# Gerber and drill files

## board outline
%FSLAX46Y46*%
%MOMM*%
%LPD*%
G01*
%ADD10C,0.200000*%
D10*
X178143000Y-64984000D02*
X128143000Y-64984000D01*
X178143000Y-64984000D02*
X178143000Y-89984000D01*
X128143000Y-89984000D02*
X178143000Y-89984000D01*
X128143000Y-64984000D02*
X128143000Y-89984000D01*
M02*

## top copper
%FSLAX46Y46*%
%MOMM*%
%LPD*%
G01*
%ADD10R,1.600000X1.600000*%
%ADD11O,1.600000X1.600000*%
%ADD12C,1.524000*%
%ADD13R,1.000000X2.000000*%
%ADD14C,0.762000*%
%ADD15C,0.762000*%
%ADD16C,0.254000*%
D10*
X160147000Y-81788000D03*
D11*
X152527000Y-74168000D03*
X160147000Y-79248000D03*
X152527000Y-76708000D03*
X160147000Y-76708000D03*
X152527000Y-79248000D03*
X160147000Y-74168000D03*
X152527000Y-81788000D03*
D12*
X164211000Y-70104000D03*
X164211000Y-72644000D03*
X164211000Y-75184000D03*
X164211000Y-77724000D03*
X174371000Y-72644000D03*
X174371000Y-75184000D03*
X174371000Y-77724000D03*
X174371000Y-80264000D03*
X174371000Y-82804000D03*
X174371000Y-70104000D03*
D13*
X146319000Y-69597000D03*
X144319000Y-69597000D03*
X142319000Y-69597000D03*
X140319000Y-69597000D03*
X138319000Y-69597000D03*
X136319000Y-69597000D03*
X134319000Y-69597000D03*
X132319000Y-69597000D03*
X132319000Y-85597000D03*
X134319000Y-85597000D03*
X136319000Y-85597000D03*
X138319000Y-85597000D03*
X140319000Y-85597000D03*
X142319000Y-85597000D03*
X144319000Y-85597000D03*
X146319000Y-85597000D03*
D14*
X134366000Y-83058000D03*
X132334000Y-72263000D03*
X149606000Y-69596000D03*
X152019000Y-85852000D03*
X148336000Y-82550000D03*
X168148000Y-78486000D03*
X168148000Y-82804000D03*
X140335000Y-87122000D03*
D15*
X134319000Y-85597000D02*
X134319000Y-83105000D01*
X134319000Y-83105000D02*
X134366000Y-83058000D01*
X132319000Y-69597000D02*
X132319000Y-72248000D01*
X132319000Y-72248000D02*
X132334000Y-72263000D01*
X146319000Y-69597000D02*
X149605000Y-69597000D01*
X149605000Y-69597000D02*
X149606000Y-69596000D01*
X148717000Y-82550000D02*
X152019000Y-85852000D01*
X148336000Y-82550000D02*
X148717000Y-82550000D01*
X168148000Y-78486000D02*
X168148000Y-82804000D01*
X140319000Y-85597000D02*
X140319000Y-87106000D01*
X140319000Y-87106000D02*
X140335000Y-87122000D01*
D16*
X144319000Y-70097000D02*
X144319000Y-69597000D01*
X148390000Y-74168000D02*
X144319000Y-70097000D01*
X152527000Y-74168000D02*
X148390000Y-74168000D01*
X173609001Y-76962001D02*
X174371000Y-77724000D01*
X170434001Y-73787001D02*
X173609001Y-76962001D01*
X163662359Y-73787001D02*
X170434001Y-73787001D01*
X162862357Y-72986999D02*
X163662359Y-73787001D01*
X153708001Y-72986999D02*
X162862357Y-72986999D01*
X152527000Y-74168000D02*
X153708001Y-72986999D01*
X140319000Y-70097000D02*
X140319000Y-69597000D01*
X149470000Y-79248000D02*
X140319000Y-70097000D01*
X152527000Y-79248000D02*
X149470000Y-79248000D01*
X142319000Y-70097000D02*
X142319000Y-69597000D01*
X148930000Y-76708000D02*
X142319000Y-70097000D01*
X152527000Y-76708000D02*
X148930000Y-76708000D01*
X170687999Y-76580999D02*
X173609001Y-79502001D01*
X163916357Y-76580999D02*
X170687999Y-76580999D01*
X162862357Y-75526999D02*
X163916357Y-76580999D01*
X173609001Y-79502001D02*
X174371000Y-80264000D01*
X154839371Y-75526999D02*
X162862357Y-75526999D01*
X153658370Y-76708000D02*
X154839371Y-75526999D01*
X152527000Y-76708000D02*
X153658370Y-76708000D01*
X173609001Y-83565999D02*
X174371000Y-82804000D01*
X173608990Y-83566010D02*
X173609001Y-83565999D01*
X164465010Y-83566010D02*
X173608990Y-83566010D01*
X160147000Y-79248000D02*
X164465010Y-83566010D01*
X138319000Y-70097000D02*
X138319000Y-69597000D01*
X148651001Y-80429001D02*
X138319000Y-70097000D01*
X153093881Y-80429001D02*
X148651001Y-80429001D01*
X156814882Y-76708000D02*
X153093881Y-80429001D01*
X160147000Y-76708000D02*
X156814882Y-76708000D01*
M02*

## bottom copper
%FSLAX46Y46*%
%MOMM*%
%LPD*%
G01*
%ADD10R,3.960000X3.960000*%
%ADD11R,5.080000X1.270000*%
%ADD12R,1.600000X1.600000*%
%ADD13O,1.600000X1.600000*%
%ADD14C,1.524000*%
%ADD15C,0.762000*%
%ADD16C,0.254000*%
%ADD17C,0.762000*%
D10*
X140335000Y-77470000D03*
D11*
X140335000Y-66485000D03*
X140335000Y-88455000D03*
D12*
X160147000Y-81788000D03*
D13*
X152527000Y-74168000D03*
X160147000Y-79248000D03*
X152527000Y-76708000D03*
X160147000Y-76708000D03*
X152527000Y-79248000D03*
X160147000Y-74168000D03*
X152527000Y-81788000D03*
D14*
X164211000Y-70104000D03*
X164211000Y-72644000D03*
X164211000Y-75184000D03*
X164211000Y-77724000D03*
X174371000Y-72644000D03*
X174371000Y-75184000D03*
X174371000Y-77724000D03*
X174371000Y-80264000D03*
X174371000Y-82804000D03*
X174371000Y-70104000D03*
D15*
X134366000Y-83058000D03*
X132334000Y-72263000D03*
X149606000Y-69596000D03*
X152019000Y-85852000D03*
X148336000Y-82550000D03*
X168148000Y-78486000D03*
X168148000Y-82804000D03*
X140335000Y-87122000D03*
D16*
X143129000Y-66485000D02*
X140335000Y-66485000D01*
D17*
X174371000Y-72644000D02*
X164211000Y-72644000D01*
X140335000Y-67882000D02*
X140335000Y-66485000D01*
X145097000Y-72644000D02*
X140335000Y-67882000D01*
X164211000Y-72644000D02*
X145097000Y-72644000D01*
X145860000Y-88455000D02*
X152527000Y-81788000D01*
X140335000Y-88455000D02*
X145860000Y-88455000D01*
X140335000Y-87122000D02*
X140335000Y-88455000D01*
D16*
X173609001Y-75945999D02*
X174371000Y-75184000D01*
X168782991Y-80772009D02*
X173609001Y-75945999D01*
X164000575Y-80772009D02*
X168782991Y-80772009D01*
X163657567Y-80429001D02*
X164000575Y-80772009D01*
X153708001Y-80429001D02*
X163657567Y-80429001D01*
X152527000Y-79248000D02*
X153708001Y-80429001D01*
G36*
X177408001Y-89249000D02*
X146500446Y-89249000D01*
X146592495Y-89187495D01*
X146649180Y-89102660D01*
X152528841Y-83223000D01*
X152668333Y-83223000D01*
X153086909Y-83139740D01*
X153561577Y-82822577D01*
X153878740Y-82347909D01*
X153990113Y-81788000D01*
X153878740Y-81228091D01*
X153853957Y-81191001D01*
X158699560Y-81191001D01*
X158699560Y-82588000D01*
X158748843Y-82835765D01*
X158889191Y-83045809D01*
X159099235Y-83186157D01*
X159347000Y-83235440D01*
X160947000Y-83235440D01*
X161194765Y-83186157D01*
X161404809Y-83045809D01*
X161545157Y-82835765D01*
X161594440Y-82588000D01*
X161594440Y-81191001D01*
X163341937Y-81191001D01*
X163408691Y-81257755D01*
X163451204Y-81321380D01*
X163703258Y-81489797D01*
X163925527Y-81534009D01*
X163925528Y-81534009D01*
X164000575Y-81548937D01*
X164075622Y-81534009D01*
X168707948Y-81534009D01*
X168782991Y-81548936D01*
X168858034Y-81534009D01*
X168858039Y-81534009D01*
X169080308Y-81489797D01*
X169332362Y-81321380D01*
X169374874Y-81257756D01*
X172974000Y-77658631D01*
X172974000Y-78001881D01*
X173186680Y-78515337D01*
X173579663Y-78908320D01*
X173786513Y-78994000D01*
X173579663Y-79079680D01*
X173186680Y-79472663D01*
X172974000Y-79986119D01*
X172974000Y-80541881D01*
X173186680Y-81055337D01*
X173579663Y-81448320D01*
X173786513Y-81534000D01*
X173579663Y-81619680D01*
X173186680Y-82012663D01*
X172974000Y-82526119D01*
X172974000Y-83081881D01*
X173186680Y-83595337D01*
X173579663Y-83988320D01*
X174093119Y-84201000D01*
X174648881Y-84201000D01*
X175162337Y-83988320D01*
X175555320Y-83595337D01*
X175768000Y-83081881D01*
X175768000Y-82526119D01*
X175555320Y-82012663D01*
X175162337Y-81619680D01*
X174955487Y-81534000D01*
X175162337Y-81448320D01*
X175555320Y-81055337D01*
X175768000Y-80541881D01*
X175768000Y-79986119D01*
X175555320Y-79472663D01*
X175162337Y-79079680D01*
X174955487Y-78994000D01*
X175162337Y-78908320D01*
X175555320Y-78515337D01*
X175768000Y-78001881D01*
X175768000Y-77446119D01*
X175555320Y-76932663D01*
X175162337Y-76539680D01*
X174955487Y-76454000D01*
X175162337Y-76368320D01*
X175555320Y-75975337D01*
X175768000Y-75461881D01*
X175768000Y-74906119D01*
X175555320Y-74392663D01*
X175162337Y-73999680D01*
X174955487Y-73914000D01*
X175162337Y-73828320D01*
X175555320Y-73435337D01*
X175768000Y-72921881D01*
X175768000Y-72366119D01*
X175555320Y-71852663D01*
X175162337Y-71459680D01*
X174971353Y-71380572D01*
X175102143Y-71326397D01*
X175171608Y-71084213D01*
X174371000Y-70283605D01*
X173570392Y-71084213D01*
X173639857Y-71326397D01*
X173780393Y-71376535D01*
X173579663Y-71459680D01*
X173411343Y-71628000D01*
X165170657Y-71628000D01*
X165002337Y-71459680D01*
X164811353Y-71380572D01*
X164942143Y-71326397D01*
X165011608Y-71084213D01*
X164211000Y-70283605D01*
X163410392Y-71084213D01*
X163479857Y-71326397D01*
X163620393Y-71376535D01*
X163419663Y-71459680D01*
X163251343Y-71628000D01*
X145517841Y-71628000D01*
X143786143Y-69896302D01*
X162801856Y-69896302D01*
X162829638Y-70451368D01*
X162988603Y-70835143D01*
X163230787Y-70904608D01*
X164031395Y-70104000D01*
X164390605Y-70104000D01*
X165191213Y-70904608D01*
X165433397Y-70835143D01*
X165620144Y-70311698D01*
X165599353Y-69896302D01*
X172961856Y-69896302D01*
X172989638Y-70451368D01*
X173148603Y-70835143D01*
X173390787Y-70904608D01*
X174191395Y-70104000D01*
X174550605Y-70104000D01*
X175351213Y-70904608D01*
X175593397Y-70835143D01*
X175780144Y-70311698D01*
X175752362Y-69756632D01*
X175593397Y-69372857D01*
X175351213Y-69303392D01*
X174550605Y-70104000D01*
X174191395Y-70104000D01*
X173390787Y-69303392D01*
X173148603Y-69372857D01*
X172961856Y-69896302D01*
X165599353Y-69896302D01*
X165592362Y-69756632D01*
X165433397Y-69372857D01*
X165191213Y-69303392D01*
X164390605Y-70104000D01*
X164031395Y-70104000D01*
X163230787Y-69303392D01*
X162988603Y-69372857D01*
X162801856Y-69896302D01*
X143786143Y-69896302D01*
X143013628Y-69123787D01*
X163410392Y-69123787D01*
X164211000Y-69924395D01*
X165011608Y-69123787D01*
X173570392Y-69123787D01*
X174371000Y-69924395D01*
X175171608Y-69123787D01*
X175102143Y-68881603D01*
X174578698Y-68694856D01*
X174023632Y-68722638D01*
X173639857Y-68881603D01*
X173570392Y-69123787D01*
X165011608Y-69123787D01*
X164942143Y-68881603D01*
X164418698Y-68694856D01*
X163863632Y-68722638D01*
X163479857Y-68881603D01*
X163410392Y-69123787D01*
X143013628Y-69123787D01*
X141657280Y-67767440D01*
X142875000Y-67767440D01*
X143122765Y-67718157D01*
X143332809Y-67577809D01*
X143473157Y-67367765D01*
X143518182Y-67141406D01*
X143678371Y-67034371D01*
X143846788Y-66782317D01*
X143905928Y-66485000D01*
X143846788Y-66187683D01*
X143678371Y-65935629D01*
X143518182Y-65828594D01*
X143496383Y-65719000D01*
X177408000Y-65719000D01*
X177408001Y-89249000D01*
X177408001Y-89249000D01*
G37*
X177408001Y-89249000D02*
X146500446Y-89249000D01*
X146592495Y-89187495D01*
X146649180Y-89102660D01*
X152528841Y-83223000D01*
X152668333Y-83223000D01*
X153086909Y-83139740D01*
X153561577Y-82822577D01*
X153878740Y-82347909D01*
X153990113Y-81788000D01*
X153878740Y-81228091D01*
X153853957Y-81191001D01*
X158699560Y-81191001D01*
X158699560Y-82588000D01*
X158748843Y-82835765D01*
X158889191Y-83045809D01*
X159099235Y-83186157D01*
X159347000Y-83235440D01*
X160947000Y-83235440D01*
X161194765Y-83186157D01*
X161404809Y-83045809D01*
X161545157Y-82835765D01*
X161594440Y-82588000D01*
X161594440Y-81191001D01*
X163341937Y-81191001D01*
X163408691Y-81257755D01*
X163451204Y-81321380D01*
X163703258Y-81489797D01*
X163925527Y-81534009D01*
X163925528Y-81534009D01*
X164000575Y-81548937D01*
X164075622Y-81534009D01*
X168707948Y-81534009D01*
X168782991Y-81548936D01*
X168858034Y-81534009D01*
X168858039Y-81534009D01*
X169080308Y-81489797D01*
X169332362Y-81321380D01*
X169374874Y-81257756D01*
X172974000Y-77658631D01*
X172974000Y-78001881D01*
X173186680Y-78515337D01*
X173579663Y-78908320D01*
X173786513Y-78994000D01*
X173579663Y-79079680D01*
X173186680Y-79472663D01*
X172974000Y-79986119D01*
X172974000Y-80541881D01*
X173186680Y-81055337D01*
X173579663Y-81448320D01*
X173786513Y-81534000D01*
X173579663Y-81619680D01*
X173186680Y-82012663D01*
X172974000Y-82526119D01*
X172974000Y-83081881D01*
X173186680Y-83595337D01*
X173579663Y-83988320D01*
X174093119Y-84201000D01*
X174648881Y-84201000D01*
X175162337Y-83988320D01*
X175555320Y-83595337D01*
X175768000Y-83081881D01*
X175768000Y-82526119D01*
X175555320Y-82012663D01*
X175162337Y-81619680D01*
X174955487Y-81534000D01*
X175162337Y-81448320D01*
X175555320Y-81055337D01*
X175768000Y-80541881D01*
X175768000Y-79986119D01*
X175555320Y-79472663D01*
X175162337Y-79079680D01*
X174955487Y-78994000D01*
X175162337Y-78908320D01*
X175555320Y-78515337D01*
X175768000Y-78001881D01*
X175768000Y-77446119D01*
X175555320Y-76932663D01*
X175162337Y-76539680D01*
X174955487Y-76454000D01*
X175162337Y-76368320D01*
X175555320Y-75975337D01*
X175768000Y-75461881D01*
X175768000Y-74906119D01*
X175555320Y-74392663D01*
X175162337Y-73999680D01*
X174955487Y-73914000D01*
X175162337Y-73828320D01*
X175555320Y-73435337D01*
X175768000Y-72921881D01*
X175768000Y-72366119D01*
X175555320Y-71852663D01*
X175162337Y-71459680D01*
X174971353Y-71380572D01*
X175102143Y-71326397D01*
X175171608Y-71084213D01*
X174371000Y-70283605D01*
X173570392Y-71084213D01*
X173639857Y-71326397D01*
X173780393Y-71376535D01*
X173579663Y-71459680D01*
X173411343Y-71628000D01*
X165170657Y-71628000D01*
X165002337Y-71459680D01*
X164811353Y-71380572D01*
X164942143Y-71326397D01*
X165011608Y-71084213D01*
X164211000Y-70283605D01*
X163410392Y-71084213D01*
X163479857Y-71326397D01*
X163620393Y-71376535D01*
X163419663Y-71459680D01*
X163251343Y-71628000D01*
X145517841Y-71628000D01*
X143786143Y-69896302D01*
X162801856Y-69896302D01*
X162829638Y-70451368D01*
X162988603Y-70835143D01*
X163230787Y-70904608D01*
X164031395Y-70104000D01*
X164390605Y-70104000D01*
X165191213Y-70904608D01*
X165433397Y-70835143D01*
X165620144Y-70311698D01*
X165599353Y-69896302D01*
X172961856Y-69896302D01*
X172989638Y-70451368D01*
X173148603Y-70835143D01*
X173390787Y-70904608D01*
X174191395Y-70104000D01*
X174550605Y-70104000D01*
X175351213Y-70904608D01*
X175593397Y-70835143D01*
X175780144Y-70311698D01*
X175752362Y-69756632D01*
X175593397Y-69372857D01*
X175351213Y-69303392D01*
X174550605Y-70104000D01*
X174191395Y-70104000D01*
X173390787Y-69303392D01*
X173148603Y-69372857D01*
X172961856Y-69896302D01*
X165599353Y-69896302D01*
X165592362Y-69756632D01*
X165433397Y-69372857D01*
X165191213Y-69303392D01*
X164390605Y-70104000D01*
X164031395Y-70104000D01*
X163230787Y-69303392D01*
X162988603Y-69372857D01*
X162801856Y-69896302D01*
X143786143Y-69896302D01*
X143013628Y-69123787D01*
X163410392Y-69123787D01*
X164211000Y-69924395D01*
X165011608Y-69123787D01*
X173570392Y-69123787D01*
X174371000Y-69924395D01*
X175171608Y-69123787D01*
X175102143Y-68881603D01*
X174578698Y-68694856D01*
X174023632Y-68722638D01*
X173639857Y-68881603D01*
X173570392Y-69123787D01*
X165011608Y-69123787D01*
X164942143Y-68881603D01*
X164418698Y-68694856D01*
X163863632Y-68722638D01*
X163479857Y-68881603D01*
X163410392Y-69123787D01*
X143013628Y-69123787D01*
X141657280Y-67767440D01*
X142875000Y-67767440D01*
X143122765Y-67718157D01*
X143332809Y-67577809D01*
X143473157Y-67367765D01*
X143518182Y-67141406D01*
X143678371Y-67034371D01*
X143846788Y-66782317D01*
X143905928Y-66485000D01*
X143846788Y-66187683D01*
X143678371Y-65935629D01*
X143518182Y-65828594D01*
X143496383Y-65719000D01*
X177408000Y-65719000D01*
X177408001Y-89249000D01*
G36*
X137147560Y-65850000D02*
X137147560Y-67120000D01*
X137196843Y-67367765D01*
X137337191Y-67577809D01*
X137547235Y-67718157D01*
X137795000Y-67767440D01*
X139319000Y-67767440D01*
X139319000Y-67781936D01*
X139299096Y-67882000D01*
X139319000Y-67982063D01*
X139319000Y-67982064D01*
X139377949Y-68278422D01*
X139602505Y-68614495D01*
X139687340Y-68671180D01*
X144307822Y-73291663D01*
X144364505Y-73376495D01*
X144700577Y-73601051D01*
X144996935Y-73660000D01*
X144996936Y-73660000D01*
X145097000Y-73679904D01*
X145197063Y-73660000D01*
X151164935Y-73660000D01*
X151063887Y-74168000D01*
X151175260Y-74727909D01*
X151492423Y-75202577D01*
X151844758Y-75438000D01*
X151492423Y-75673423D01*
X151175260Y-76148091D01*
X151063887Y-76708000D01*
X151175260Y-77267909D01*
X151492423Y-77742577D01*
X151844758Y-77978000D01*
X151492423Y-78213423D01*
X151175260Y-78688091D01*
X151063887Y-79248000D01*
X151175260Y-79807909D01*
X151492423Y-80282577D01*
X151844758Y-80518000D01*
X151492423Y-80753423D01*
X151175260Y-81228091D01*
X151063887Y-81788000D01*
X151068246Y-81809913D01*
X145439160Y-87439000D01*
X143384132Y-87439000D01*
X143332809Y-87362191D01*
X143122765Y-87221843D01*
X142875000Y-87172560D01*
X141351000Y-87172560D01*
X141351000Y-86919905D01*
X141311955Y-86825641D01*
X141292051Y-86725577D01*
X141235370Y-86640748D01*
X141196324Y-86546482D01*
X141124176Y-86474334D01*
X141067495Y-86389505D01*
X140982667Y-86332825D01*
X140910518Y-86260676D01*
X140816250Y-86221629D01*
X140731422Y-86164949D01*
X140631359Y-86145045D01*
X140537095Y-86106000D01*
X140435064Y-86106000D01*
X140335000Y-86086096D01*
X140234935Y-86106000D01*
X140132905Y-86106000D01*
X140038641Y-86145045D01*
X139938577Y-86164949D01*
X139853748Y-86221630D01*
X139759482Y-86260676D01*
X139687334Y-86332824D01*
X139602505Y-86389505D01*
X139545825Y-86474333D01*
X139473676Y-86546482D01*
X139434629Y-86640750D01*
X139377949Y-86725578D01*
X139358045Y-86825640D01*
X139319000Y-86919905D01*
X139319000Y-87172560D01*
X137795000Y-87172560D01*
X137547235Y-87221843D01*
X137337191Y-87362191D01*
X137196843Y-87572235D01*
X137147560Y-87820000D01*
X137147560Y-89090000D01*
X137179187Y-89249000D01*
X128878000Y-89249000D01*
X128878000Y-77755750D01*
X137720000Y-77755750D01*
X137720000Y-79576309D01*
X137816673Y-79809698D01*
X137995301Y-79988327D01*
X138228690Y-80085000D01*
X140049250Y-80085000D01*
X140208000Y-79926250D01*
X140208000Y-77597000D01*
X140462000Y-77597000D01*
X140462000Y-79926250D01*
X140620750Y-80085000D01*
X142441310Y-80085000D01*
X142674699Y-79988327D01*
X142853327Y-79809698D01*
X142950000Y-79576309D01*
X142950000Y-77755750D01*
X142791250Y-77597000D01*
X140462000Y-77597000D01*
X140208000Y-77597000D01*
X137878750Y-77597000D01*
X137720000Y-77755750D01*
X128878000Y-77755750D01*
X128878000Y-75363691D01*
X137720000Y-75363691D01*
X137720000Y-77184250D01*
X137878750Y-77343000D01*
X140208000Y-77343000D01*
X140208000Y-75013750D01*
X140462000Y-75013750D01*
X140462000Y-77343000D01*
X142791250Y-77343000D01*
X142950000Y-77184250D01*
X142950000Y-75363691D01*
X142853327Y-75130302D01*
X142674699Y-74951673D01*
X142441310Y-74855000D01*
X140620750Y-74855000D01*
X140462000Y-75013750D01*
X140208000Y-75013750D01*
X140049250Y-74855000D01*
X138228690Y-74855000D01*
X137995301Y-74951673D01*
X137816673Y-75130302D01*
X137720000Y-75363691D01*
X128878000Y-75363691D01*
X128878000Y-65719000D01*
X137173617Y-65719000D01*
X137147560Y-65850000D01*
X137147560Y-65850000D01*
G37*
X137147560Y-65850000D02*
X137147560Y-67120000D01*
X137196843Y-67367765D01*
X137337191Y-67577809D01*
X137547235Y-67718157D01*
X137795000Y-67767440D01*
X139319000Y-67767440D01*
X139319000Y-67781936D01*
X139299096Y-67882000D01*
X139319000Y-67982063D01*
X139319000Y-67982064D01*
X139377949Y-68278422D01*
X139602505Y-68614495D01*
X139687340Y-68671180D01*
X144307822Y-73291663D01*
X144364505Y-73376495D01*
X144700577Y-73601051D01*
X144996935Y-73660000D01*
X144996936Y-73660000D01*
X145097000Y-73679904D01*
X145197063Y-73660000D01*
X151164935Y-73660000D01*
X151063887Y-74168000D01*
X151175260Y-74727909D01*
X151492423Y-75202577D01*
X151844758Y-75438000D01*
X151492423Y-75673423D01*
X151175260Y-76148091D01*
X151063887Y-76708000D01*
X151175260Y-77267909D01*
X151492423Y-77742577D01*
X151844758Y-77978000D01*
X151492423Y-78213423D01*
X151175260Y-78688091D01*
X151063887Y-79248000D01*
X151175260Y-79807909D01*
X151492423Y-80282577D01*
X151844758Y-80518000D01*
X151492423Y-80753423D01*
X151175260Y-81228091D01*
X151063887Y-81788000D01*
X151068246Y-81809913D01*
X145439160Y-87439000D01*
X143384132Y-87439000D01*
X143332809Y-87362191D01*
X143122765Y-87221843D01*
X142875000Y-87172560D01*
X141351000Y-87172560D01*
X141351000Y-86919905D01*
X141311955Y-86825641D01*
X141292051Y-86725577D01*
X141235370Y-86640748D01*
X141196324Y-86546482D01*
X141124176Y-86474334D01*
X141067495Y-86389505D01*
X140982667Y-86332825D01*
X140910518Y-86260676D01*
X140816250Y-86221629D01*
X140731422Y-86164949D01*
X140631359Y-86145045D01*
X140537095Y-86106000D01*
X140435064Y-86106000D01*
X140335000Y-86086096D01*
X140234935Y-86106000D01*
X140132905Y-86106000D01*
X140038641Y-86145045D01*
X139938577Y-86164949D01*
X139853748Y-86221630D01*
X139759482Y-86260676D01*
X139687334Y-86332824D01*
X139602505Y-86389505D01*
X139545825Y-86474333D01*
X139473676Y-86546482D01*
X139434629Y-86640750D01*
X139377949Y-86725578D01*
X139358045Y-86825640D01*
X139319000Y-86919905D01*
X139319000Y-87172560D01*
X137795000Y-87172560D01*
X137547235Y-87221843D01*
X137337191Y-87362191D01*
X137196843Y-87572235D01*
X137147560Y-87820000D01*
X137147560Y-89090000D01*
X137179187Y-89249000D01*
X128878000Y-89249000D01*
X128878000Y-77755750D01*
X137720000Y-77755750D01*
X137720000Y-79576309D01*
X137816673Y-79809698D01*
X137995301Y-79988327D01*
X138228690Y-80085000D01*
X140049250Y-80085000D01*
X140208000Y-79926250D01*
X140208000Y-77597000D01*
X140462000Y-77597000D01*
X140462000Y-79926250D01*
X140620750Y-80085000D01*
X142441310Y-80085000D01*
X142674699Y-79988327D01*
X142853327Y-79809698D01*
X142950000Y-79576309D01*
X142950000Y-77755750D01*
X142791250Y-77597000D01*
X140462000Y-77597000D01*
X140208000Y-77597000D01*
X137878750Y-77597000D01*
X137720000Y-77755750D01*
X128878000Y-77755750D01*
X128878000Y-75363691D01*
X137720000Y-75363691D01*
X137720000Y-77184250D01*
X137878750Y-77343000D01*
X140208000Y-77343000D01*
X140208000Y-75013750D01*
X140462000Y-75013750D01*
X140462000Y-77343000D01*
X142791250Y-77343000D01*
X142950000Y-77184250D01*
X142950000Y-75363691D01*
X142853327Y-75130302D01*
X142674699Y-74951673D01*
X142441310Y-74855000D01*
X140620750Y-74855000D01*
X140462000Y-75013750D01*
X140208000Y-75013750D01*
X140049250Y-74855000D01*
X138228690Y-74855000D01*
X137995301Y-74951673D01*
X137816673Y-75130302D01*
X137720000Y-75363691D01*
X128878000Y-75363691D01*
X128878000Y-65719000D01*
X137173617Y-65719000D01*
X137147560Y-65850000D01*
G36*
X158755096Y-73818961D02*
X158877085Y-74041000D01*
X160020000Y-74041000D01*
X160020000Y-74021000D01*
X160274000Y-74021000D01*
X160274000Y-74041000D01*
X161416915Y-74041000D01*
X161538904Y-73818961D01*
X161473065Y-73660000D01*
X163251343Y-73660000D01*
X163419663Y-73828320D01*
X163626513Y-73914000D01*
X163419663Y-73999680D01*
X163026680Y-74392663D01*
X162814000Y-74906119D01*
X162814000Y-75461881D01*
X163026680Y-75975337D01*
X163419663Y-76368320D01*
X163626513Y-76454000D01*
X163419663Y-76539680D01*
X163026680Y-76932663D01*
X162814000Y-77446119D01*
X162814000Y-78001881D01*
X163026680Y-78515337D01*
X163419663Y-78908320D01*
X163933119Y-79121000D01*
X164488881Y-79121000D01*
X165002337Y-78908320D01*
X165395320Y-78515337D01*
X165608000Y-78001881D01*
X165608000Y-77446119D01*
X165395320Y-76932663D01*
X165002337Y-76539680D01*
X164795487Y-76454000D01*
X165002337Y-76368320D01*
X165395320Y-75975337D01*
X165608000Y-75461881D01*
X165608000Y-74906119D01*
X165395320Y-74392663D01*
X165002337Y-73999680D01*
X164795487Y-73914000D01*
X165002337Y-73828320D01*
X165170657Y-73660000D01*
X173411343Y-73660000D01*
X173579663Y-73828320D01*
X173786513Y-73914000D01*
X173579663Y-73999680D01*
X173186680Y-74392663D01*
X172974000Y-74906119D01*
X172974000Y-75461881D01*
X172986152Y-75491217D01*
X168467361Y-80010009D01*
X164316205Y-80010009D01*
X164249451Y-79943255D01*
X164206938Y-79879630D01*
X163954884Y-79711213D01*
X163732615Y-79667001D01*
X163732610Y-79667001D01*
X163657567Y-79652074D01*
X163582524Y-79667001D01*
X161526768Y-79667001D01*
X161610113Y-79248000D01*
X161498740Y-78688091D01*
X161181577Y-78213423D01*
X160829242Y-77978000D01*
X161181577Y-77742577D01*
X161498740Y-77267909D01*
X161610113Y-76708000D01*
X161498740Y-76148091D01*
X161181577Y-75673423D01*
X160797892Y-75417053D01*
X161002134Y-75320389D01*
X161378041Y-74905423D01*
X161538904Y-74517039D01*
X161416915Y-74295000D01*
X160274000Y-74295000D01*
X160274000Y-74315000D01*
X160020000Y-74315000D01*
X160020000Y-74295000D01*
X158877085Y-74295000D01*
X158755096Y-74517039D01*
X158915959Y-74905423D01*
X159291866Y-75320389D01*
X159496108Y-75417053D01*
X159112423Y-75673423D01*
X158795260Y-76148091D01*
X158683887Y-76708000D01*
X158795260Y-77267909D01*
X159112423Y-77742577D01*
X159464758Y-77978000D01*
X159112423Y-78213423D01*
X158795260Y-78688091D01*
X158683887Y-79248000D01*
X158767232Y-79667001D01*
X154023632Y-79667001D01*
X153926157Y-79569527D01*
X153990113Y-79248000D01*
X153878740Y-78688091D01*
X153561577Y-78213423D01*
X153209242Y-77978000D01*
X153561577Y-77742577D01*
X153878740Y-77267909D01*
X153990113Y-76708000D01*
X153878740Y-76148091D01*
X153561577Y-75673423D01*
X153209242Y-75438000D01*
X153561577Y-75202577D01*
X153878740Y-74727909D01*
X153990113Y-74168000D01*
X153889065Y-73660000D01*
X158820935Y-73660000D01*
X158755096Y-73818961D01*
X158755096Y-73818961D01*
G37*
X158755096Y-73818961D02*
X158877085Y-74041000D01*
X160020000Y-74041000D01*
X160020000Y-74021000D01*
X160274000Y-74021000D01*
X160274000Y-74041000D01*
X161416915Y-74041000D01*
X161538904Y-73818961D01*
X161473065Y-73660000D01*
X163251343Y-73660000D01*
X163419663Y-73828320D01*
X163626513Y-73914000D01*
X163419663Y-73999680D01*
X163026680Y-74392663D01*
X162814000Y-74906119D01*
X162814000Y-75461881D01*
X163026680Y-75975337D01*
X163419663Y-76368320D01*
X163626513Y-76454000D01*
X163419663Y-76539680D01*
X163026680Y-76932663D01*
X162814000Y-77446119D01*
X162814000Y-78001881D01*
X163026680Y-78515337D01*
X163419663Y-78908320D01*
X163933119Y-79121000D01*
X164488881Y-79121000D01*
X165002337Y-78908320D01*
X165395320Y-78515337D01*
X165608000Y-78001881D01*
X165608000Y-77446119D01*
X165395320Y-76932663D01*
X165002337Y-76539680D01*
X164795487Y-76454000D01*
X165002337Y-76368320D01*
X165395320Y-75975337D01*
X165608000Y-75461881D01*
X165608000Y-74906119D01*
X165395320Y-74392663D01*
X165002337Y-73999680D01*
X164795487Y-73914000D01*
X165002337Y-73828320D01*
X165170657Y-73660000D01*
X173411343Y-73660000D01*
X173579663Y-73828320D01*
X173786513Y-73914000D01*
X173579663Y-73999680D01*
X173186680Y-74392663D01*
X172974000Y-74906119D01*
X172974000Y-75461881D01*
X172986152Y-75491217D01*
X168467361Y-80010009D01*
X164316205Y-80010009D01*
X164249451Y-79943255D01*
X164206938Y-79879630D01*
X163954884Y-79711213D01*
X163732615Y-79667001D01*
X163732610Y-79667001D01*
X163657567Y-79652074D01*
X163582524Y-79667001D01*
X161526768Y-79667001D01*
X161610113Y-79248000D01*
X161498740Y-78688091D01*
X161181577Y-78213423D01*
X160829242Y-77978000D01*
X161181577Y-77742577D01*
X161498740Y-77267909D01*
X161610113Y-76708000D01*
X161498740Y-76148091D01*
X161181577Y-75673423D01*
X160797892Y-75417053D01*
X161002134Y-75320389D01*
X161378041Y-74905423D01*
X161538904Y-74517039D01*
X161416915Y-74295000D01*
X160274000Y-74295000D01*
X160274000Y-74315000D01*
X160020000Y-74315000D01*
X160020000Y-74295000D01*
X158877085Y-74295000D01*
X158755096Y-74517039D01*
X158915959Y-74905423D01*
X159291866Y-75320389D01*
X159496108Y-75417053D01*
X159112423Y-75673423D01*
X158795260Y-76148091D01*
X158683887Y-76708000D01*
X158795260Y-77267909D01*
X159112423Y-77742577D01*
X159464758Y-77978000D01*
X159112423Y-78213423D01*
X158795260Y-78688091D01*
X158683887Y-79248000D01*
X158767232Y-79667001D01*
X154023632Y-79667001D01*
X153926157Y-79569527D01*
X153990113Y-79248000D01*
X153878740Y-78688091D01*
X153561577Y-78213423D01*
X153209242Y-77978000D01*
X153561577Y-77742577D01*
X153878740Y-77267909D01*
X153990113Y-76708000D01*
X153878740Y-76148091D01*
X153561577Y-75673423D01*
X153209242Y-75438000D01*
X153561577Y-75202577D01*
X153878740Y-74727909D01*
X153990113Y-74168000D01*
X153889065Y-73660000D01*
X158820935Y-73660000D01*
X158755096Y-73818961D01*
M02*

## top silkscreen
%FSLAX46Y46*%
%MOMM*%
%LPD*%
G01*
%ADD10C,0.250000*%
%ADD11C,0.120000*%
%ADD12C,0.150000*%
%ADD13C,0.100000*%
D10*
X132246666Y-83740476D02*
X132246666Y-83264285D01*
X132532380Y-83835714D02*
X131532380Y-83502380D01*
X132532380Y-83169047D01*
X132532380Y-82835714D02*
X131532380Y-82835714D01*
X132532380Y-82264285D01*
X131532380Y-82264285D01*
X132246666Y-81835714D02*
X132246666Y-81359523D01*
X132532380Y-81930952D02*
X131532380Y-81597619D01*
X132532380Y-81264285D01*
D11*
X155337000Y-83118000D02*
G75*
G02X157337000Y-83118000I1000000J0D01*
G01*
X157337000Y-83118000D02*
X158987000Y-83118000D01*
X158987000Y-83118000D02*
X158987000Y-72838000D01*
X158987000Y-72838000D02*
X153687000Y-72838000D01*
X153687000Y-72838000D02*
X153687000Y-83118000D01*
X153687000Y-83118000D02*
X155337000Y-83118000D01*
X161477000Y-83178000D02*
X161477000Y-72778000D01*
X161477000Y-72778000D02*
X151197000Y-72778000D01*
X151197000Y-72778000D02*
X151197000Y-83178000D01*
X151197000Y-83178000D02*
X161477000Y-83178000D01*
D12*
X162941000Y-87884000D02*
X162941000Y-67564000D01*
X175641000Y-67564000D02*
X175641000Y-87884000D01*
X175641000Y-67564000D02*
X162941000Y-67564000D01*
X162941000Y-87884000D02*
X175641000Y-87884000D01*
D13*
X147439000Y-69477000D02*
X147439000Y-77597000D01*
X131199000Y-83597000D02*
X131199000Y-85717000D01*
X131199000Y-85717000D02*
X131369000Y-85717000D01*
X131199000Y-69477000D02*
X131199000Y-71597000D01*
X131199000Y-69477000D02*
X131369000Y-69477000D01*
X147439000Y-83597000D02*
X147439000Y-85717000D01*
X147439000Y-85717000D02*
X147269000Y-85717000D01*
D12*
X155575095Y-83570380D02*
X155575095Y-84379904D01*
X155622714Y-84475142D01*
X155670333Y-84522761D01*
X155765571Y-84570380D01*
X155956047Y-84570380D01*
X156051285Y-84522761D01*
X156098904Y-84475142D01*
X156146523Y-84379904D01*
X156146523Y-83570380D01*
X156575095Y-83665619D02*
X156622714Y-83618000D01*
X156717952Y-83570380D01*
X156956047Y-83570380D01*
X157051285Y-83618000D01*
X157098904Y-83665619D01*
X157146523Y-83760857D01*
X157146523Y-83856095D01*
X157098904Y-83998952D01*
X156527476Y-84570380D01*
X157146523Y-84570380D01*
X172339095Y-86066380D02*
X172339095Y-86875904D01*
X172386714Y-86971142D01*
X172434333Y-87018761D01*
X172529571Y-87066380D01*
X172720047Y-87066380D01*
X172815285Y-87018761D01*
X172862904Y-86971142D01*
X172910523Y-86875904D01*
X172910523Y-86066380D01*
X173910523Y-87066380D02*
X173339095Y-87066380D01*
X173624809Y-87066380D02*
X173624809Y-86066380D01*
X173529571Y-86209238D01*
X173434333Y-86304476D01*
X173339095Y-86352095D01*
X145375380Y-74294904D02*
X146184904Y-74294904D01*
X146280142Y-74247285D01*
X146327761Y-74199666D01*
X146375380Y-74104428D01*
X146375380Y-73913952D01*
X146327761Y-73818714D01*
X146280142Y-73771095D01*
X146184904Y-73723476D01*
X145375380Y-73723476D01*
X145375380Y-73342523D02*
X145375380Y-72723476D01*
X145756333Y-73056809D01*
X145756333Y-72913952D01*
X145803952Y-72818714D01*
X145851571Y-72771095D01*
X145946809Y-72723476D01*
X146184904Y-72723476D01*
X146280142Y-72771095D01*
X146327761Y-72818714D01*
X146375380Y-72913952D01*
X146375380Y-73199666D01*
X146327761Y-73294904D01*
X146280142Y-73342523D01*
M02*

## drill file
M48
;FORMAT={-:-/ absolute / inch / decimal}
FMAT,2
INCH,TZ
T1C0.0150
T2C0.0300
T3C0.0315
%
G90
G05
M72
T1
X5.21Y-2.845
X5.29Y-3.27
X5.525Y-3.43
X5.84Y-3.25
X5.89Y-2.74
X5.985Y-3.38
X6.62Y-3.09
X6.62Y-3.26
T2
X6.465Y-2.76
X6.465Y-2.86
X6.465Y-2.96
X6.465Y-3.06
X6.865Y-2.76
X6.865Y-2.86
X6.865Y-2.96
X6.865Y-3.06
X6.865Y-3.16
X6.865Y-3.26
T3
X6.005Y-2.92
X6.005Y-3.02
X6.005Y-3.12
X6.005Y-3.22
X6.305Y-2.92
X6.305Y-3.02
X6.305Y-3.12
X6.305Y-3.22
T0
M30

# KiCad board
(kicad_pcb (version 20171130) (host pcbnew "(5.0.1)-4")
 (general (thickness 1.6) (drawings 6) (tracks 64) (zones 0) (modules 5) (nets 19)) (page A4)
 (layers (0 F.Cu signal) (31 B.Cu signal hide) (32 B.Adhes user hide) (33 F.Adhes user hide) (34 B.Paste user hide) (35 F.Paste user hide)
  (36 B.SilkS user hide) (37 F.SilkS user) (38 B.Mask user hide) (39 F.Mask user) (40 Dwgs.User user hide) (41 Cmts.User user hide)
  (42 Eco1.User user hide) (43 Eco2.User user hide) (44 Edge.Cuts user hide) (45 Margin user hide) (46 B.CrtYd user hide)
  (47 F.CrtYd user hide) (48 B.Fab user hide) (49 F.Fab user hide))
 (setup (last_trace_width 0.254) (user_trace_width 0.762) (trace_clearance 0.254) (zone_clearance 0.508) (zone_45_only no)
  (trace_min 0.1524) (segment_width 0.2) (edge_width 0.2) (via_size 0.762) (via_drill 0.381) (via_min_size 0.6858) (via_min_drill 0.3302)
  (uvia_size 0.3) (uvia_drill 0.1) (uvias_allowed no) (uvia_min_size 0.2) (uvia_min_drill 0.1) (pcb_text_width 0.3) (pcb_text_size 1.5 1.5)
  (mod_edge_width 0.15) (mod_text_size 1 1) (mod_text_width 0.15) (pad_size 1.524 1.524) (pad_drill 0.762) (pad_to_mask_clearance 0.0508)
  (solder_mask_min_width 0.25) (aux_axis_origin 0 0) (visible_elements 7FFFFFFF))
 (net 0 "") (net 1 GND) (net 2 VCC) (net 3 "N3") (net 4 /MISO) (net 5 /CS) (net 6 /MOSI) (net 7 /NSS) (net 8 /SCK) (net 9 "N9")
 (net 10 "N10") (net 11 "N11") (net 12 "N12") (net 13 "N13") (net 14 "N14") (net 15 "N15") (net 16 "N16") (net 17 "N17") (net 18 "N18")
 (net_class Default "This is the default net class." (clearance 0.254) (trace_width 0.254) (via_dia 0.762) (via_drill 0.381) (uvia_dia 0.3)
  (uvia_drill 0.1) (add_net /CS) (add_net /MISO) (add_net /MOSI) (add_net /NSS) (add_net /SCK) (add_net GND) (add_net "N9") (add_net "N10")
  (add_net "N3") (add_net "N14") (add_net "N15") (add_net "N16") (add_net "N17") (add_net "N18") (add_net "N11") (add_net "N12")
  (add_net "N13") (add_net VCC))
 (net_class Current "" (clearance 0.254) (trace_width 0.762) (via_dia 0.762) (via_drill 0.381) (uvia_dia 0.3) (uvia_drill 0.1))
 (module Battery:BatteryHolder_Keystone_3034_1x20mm (layer B.Cu) (at 140.335 77.47 90)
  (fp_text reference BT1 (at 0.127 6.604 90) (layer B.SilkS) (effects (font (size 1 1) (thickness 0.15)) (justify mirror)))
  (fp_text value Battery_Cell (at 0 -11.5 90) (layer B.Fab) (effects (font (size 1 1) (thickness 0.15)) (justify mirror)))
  (pad 2 smd rect (at 0 0 90) (size 3.96 3.96) (layers B.Cu B.Paste B.Mask) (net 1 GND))
  (pad 1 smd rect (at 10.985 0 90) (size 1.27 5.08) (layers B.Cu B.Paste B.Mask) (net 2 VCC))
  (pad 1 smd rect (at -10.985 0 90) (size 1.27 5.08) (layers B.Cu B.Paste B.Mask) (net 2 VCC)))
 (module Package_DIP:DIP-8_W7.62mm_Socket (layer F.Cu) (at 160.147 81.788 180)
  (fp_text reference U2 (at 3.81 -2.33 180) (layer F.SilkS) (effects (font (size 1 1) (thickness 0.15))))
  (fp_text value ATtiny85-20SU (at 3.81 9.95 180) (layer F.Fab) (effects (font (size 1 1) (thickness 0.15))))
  (fp_arc (start 3.81 -1.33) (end 2.81 -1.33) (angle -180) (layer F.SilkS) (width 0.12))
  (fp_line (start 2.81 -1.33) (end 1.16 -1.33) (layer F.SilkS) (width 0.12))
  (fp_line (start 1.16 -1.33) (end 1.16 8.95) (layer F.SilkS) (width 0.12))
  (fp_line (start 1.16 8.95) (end 6.46 8.95) (layer F.SilkS) (width 0.12))
  (fp_line (start 6.46 8.95) (end 6.46 -1.33) (layer F.SilkS) (width 0.12))
  (fp_line (start 6.46 -1.33) (end 4.81 -1.33) (layer F.SilkS) (width 0.12))
  (fp_line (start -1.33 -1.39) (end -1.33 9.01) (layer F.SilkS) (width 0.12))
  (fp_line (start -1.33 9.01) (end 8.95 9.01) (layer F.SilkS) (width 0.12))
  (fp_line (start 8.95 9.01) (end 8.95 -1.39) (layer F.SilkS) (width 0.12))
  (fp_line (start 8.95 -1.39) (end -1.33 -1.39) (layer F.SilkS) (width 0.12))
  (pad 1 thru_hole rect (at 0 0 180) (size 1.6 1.6) (drill 0.8) (layers *.Cu *.Mask) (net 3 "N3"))
  (pad 5 thru_hole oval (at 7.62 7.62 180) (size 1.6 1.6) (drill 0.8) (layers *.Cu *.Mask) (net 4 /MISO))
  (pad 2 thru_hole oval (at 0 2.54 180) (size 1.6 1.6) (drill 0.8) (layers *.Cu *.Mask) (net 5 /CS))
  (pad 6 thru_hole oval (at 7.62 5.08 180) (size 1.6 1.6) (drill 0.8) (layers *.Cu *.Mask) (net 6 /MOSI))
  (pad 3 thru_hole oval (at 0 5.08 180) (size 1.6 1.6) (drill 0.8) (layers *.Cu *.Mask) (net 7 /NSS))
  (pad 7 thru_hole oval (at 7.62 2.54 180) (size 1.6 1.6) (drill 0.8) (layers *.Cu *.Mask) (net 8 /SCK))
  (pad 4 thru_hole oval (at 0 7.62 180) (size 1.6 1.6) (drill 0.8) (layers *.Cu *.Mask) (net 1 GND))
  (pad 8 thru_hole oval (at 7.62 0 180) (size 1.6 1.6) (drill 0.8) (layers *.Cu *.Mask) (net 2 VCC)))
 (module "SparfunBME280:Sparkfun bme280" (layer F.Cu) (at 169.291 77.724)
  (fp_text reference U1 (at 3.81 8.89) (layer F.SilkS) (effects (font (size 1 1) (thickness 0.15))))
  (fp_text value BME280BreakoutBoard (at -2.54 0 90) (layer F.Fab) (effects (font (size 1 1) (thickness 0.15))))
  (fp_line (start -6.35 10.16) (end -6.35 -10.16) (layer F.SilkS) (width 0.15))
  (fp_line (start 6.35 -10.16) (end 6.35 10.16) (layer F.SilkS) (width 0.15))
  (fp_line (start 6.35 -10.16) (end -6.35 -10.16) (layer F.SilkS) (width 0.15))
  (fp_line (start -6.35 10.16) (end 6.35 10.16) (layer F.SilkS) (width 0.15))
  (pad 1 thru_hole circle (at -5.08 -7.62) (size 1.524 1.524) (drill 0.762) (layers *.Cu *.Mask) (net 1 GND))
  (pad 2 thru_hole circle (at -5.08 -5.08) (size 1.524 1.524) (drill 0.762) (layers *.Cu *.Mask) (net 2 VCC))
  (pad 3 thru_hole circle (at -5.08 -2.54) (size 1.524 1.524) (drill 0.762) (layers *.Cu *.Mask) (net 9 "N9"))
  (pad 4 thru_hole circle (at -5.08 0) (size 1.524 1.524) (drill 0.762) (layers *.Cu *.Mask) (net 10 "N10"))
  (pad 6 thru_hole circle (at 5.08 -5.08) (size 1.524 1.524) (drill 0.762) (layers *.Cu *.Mask) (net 2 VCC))
  (pad 7 thru_hole circle (at 5.08 -2.54) (size 1.524 1.524) (drill 0.762) (layers *.Cu *.Mask) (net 8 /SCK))
  (pad 8 thru_hole circle (at 5.08 0) (size 1.524 1.524) (drill 0.762) (layers *.Cu *.Mask) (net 4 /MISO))
  (pad 9 thru_hole circle (at 5.08 2.54) (size 1.524 1.524) (drill 0.762) (layers *.Cu *.Mask) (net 6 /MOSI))
  (pad 10 thru_hole circle (at 5.08 5.08) (size 1.524 1.524) (drill 0.762) (layers *.Cu *.Mask) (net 5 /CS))
  (pad 5 thru_hole circle (at 5.08 -7.62) (size 1.524 1.524) (drill 0.762) (layers *.Cu *.Mask) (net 1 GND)))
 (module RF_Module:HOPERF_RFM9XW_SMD (layer F.Cu) (at 139.319 77.597 270)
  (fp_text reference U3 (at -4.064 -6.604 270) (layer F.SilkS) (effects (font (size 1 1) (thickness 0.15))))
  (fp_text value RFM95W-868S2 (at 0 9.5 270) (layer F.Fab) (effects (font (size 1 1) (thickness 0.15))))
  (fp_line (start -8.12 -8.12) (end 0 -8.12) (layer F.SilkS) (width 0.1))
  (fp_line (start 6 8.12) (end 8.12 8.12) (layer F.SilkS) (width 0.1))
  (fp_line (start 8.12 8.12) (end 8.12 7.95) (layer F.SilkS) (width 0.1))
  (fp_line (start -8.12 8.12) (end -6 8.12) (layer F.SilkS) (width 0.1))
  (fp_line (start -8.12 8.12) (end -8.12 7.95) (layer F.SilkS) (width 0.1))
  (fp_line (start 6 -8.12) (end 8.12 -8.12) (layer F.SilkS) (width 0.1))
  (fp_line (start 8.12 -8.12) (end 8.12 -7.95) (layer F.SilkS) (width 0.1))
  (pad 1 smd rect (at -8 -7 270) (size 2 1) (layers F.Cu F.Paste F.Mask) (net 1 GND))
  (pad 2 smd rect (at -8 -5 270) (size 2 1) (layers F.Cu F.Paste F.Mask) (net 4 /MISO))
  (pad 3 smd rect (at -8 -3 270) (size 2 1) (layers F.Cu F.Paste F.Mask) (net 6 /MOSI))
  (pad 4 smd rect (at -8 -1 270) (size 2 1) (layers F.Cu F.Paste F.Mask) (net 8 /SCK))
  (pad 5 smd rect (at -8 1 270) (size 2 1) (layers F.Cu F.Paste F.Mask) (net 7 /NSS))
  (pad 6 smd rect (at -8 3 270) (size 2 1) (layers F.Cu F.Paste F.Mask) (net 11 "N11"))
  (pad 7 smd rect (at -8 5 270) (size 2 1) (layers F.Cu F.Paste F.Mask) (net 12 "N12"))
  (pad 8 smd rect (at -8 7 270) (size 2 1) (layers F.Cu F.Paste F.Mask) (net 1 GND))
  (pad 9 smd rect (at 8 7 270) (size 2 1) (layers F.Cu F.Paste F.Mask) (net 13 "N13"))
  (pad 10 smd rect (at 8 5 270) (size 2 1) (layers F.Cu F.Paste F.Mask) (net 1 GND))
  (pad 11 smd rect (at 8 3 270) (size 2 1) (layers F.Cu F.Paste F.Mask) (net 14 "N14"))
  (pad 12 smd rect (at 8 1 270) (size 2 1) (layers F.Cu F.Paste F.Mask) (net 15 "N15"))
  (pad 13 smd rect (at 8 -1 270) (size 2 1) (layers F.Cu F.Paste F.Mask) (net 2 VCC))
  (pad 14 smd rect (at 8 -3 270) (size 2 1) (layers F.Cu F.Paste F.Mask) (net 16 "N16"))
  (pad 15 smd rect (at 8 -5 270) (size 2 1) (layers F.Cu F.Paste F.Mask) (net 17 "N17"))
  (pad 16 smd rect (at 8 -7 270) (size 2 1) (layers F.Cu F.Paste F.Mask) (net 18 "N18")))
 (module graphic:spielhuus (layer B.Cu) (at 171.069 68.072 270)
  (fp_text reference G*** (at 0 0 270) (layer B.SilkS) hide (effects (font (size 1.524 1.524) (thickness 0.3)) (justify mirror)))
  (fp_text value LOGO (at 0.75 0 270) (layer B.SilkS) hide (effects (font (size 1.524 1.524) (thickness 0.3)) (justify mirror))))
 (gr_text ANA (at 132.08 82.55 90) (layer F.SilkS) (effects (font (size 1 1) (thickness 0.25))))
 (gr_line (start 178.143 64.984) (end 128.143 64.984) (layer Edge.Cuts) (width 0.2))
 (gr_line (start 178.143 64.984) (end 178.143 89.984) (layer Edge.Cuts) (width 0.2))
 (gr_line (start 128.143 89.984) (end 178.143 89.984) (layer Edge.Cuts) (width 0.2))
 (gr_line (start 128.143 64.984) (end 128.143 89.984) (layer Edge.Cuts) (width 0.2))
 (via (at 134.366 83.058) (size 0.762) (drill 0.381) (layers F.Cu B.Cu) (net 1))
 (segment (start 134.319 85.597) (end 134.319 83.105) (width 0.762) (layer F.Cu) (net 1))
 (segment (start 134.319 83.105) (end 134.366 83.058) (width 0.762) (layer F.Cu) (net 1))
 (via (at 132.334 72.263) (size 0.762) (drill 0.381) (layers F.Cu B.Cu) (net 1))
 (segment (start 132.319 69.597) (end 132.319 72.248) (width 0.762) (layer F.Cu) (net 1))
 (segment (start 132.319 72.248) (end 132.334 72.263) (width 0.762) (layer F.Cu) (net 1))
 (via (at 149.606 69.596) (size 0.762) (drill 0.381) (layers F.Cu B.Cu) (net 1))
 (segment (start 146.319 69.597) (end 149.605 69.597) (width 0.762) (layer F.Cu) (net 1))
 (segment (start 149.605 69.597) (end 149.606 69.596) (width 0.762) (layer F.Cu) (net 1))
 (via (at 152.019 85.852) (size 0.762) (drill 0.381) (layers F.Cu B.Cu) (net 1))
 (via (at 148.336 82.55) (size 0.762) (drill 0.381) (layers F.Cu B.Cu) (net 1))
 (segment (start 148.717 82.55) (end 152.019 85.852) (width 0.762) (layer F.Cu) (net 1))
 (segment (start 148.336 82.55) (end 148.717 82.55) (width 0.762) (layer F.Cu) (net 1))
 (via (at 168.148 78.486) (size 0.762) (drill 0.381) (layers F.Cu B.Cu) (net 1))
 (via (at 168.148 82.804) (size 0.762) (drill 0.381) (layers F.Cu B.Cu) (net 1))
 (segment (start 168.148 78.486) (end 168.148 82.804) (width 0.762) (layer F.Cu) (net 1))
 (segment (start 143.129 66.485) (end 140.335 66.485) (width 0.254) (layer B.Cu) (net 2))
 (segment (start 174.371 72.644) (end 164.211 72.644) (width 0.762) (layer B.Cu) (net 2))
 (segment (start 140.335 67.882) (end 140.335 66.485) (width 0.762) (layer B.Cu) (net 2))
 (segment (start 145.097 72.644) (end 140.335 67.882) (width 0.762) (layer B.Cu) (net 2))
 (segment (start 164.211 72.644) (end 145.097 72.644) (width 0.762) (layer B.Cu) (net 2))
 (segment (start 145.86 88.455) (end 152.527 81.788) (width 0.762) (layer B.Cu) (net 2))
 (segment (start 140.335 88.455) (end 145.86 88.455) (width 0.762) (layer B.Cu) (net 2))
 (via (at 140.335 87.122) (size 0.762) (drill 0.381) (layers F.Cu B.Cu) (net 2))
 (segment (start 140.319 85.597) (end 140.319 87.106) (width 0.762) (layer F.Cu) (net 2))
 (segment (start 140.319 87.106) (end 140.335 87.122) (width 0.762) (layer F.Cu) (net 2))
 (segment (start 140.335 87.122) (end 140.335 88.455) (width 0.762) (layer B.Cu) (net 2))
 (segment (start 144.319 70.097) (end 144.319 69.597) (width 0.254) (layer F.Cu) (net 4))
 (segment (start 148.39 74.168) (end 144.319 70.097) (width 0.254) (layer F.Cu) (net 4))
 (segment (start 152.527 74.168) (end 148.39 74.168) (width 0.254) (layer F.Cu) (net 4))
 (segment (start 173.609001 76.962001) (end 174.371 77.724) (width 0.254) (layer F.Cu) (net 4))
 (segment (start 170.434001 73.787001) (end 173.609001 76.962001) (width 0.254) (layer F.Cu) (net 4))
 (segment (start 163.662359 73.787001) (end 170.434001 73.787001) (width 0.254) (layer F.Cu) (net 4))
 (segment (start 162.862357 72.986999) (end 163.662359 73.787001) (width 0.254) (layer F.Cu) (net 4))
 (segment (start 153.708001 72.986999) (end 162.862357 72.986999) (width 0.254) (layer F.Cu) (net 4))
 (segment (start 152.527 74.168) (end 153.708001 72.986999) (width 0.254) (layer F.Cu) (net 4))
 (segment (start 140.319 70.097) (end 140.319 69.597) (width 0.254) (layer F.Cu) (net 8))
 (segment (start 149.47 79.248) (end 140.319 70.097) (width 0.254) (layer F.Cu) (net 8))
 (segment (start 152.527 79.248) (end 149.47 79.248) (width 0.254) (layer F.Cu) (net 8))
 (segment (start 173.609001 75.945999) (end 174.371 75.184) (width 0.254) (layer B.Cu) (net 8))
 (segment (start 168.782991 80.772009) (end 173.609001 75.945999) (width 0.254) (layer B.Cu) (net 8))
 (segment (start 164.000575 80.772009) (end 168.782991 80.772009) (width 0.254) (layer B.Cu) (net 8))
 (segment (start 163.657567 80.429001) (end 164.000575 80.772009) (width 0.254) (layer B.Cu) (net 8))
 (segment (start 153.708001 80.429001) (end 163.657567 80.429001) (width 0.254) (layer B.Cu) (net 8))
 (segment (start 152.527 79.248) (end 153.708001 80.429001) (width 0.254) (layer B.Cu) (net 8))
 (segment (start 142.319 70.097) (end 142.319 69.597) (width 0.254) (layer F.Cu) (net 6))
 (segment (start 148.93 76.708) (end 142.319 70.097) (width 0.254) (layer F.Cu) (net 6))
 (segment (start 152.527 76.708) (end 148.93 76.708) (width 0.254) (layer F.Cu) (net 6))
 (segment (start 170.687999 76.580999) (end 173.609001 79.502001) (width 0.254) (layer F.Cu) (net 6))
 (segment (start 163.916357 76.580999) (end 170.687999 76.580999) (width 0.254) (layer F.Cu) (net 6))
 (segment (start 162.862357 75.526999) (end 163.916357 76.580999) (width 0.254) (layer F.Cu) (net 6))
 (segment (start 173.609001 79.502001) (end 174.371 80.264) (width 0.254) (layer F.Cu) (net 6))
 (segment (start 154.839371 75.526999) (end 162.862357 75.526999) (width 0.254) (layer F.Cu) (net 6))
 (segment (start 153.65837 76.708) (end 154.839371 75.526999) (width 0.254) (layer F.Cu) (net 6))
 (segment (start 152.527 76.708) (end 153.65837 76.708) (width 0.254) (layer F.Cu) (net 6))
 (segment (start 173.609001 83.565999) (end 174.371 82.804) (width 0.254) (layer F.Cu) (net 5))
 (segment (start 173.60899 83.56601) (end 173.609001 83.565999) (width 0.254) (layer F.Cu) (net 5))
 (segment (start 164.46501 83.56601) (end 173.60899 83.56601) (width 0.254) (layer F.Cu) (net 5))
 (segment (start 160.147 79.248) (end 164.46501 83.56601) (width 0.254) (layer F.Cu) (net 5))
 (segment (start 138.319 70.097) (end 138.319 69.597) (width 0.254) (layer F.Cu) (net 7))
 (segment (start 148.651001 80.429001) (end 138.319 70.097) (width 0.254) (layer F.Cu) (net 7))
 (segment (start 153.093881 80.429001) (end 148.651001 80.429001) (width 0.254) (layer F.Cu) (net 7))
 (segment (start 156.814882 76.708) (end 153.093881 80.429001) (width 0.254) (layer F.Cu) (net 7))
 (segment (start 160.147 76.708) (end 156.814882 76.708) (width 0.254) (layer F.Cu) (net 7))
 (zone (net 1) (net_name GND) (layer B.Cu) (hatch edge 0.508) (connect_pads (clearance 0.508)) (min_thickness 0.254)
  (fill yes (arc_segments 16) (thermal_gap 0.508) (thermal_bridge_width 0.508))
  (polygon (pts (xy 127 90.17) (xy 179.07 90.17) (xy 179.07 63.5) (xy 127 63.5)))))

